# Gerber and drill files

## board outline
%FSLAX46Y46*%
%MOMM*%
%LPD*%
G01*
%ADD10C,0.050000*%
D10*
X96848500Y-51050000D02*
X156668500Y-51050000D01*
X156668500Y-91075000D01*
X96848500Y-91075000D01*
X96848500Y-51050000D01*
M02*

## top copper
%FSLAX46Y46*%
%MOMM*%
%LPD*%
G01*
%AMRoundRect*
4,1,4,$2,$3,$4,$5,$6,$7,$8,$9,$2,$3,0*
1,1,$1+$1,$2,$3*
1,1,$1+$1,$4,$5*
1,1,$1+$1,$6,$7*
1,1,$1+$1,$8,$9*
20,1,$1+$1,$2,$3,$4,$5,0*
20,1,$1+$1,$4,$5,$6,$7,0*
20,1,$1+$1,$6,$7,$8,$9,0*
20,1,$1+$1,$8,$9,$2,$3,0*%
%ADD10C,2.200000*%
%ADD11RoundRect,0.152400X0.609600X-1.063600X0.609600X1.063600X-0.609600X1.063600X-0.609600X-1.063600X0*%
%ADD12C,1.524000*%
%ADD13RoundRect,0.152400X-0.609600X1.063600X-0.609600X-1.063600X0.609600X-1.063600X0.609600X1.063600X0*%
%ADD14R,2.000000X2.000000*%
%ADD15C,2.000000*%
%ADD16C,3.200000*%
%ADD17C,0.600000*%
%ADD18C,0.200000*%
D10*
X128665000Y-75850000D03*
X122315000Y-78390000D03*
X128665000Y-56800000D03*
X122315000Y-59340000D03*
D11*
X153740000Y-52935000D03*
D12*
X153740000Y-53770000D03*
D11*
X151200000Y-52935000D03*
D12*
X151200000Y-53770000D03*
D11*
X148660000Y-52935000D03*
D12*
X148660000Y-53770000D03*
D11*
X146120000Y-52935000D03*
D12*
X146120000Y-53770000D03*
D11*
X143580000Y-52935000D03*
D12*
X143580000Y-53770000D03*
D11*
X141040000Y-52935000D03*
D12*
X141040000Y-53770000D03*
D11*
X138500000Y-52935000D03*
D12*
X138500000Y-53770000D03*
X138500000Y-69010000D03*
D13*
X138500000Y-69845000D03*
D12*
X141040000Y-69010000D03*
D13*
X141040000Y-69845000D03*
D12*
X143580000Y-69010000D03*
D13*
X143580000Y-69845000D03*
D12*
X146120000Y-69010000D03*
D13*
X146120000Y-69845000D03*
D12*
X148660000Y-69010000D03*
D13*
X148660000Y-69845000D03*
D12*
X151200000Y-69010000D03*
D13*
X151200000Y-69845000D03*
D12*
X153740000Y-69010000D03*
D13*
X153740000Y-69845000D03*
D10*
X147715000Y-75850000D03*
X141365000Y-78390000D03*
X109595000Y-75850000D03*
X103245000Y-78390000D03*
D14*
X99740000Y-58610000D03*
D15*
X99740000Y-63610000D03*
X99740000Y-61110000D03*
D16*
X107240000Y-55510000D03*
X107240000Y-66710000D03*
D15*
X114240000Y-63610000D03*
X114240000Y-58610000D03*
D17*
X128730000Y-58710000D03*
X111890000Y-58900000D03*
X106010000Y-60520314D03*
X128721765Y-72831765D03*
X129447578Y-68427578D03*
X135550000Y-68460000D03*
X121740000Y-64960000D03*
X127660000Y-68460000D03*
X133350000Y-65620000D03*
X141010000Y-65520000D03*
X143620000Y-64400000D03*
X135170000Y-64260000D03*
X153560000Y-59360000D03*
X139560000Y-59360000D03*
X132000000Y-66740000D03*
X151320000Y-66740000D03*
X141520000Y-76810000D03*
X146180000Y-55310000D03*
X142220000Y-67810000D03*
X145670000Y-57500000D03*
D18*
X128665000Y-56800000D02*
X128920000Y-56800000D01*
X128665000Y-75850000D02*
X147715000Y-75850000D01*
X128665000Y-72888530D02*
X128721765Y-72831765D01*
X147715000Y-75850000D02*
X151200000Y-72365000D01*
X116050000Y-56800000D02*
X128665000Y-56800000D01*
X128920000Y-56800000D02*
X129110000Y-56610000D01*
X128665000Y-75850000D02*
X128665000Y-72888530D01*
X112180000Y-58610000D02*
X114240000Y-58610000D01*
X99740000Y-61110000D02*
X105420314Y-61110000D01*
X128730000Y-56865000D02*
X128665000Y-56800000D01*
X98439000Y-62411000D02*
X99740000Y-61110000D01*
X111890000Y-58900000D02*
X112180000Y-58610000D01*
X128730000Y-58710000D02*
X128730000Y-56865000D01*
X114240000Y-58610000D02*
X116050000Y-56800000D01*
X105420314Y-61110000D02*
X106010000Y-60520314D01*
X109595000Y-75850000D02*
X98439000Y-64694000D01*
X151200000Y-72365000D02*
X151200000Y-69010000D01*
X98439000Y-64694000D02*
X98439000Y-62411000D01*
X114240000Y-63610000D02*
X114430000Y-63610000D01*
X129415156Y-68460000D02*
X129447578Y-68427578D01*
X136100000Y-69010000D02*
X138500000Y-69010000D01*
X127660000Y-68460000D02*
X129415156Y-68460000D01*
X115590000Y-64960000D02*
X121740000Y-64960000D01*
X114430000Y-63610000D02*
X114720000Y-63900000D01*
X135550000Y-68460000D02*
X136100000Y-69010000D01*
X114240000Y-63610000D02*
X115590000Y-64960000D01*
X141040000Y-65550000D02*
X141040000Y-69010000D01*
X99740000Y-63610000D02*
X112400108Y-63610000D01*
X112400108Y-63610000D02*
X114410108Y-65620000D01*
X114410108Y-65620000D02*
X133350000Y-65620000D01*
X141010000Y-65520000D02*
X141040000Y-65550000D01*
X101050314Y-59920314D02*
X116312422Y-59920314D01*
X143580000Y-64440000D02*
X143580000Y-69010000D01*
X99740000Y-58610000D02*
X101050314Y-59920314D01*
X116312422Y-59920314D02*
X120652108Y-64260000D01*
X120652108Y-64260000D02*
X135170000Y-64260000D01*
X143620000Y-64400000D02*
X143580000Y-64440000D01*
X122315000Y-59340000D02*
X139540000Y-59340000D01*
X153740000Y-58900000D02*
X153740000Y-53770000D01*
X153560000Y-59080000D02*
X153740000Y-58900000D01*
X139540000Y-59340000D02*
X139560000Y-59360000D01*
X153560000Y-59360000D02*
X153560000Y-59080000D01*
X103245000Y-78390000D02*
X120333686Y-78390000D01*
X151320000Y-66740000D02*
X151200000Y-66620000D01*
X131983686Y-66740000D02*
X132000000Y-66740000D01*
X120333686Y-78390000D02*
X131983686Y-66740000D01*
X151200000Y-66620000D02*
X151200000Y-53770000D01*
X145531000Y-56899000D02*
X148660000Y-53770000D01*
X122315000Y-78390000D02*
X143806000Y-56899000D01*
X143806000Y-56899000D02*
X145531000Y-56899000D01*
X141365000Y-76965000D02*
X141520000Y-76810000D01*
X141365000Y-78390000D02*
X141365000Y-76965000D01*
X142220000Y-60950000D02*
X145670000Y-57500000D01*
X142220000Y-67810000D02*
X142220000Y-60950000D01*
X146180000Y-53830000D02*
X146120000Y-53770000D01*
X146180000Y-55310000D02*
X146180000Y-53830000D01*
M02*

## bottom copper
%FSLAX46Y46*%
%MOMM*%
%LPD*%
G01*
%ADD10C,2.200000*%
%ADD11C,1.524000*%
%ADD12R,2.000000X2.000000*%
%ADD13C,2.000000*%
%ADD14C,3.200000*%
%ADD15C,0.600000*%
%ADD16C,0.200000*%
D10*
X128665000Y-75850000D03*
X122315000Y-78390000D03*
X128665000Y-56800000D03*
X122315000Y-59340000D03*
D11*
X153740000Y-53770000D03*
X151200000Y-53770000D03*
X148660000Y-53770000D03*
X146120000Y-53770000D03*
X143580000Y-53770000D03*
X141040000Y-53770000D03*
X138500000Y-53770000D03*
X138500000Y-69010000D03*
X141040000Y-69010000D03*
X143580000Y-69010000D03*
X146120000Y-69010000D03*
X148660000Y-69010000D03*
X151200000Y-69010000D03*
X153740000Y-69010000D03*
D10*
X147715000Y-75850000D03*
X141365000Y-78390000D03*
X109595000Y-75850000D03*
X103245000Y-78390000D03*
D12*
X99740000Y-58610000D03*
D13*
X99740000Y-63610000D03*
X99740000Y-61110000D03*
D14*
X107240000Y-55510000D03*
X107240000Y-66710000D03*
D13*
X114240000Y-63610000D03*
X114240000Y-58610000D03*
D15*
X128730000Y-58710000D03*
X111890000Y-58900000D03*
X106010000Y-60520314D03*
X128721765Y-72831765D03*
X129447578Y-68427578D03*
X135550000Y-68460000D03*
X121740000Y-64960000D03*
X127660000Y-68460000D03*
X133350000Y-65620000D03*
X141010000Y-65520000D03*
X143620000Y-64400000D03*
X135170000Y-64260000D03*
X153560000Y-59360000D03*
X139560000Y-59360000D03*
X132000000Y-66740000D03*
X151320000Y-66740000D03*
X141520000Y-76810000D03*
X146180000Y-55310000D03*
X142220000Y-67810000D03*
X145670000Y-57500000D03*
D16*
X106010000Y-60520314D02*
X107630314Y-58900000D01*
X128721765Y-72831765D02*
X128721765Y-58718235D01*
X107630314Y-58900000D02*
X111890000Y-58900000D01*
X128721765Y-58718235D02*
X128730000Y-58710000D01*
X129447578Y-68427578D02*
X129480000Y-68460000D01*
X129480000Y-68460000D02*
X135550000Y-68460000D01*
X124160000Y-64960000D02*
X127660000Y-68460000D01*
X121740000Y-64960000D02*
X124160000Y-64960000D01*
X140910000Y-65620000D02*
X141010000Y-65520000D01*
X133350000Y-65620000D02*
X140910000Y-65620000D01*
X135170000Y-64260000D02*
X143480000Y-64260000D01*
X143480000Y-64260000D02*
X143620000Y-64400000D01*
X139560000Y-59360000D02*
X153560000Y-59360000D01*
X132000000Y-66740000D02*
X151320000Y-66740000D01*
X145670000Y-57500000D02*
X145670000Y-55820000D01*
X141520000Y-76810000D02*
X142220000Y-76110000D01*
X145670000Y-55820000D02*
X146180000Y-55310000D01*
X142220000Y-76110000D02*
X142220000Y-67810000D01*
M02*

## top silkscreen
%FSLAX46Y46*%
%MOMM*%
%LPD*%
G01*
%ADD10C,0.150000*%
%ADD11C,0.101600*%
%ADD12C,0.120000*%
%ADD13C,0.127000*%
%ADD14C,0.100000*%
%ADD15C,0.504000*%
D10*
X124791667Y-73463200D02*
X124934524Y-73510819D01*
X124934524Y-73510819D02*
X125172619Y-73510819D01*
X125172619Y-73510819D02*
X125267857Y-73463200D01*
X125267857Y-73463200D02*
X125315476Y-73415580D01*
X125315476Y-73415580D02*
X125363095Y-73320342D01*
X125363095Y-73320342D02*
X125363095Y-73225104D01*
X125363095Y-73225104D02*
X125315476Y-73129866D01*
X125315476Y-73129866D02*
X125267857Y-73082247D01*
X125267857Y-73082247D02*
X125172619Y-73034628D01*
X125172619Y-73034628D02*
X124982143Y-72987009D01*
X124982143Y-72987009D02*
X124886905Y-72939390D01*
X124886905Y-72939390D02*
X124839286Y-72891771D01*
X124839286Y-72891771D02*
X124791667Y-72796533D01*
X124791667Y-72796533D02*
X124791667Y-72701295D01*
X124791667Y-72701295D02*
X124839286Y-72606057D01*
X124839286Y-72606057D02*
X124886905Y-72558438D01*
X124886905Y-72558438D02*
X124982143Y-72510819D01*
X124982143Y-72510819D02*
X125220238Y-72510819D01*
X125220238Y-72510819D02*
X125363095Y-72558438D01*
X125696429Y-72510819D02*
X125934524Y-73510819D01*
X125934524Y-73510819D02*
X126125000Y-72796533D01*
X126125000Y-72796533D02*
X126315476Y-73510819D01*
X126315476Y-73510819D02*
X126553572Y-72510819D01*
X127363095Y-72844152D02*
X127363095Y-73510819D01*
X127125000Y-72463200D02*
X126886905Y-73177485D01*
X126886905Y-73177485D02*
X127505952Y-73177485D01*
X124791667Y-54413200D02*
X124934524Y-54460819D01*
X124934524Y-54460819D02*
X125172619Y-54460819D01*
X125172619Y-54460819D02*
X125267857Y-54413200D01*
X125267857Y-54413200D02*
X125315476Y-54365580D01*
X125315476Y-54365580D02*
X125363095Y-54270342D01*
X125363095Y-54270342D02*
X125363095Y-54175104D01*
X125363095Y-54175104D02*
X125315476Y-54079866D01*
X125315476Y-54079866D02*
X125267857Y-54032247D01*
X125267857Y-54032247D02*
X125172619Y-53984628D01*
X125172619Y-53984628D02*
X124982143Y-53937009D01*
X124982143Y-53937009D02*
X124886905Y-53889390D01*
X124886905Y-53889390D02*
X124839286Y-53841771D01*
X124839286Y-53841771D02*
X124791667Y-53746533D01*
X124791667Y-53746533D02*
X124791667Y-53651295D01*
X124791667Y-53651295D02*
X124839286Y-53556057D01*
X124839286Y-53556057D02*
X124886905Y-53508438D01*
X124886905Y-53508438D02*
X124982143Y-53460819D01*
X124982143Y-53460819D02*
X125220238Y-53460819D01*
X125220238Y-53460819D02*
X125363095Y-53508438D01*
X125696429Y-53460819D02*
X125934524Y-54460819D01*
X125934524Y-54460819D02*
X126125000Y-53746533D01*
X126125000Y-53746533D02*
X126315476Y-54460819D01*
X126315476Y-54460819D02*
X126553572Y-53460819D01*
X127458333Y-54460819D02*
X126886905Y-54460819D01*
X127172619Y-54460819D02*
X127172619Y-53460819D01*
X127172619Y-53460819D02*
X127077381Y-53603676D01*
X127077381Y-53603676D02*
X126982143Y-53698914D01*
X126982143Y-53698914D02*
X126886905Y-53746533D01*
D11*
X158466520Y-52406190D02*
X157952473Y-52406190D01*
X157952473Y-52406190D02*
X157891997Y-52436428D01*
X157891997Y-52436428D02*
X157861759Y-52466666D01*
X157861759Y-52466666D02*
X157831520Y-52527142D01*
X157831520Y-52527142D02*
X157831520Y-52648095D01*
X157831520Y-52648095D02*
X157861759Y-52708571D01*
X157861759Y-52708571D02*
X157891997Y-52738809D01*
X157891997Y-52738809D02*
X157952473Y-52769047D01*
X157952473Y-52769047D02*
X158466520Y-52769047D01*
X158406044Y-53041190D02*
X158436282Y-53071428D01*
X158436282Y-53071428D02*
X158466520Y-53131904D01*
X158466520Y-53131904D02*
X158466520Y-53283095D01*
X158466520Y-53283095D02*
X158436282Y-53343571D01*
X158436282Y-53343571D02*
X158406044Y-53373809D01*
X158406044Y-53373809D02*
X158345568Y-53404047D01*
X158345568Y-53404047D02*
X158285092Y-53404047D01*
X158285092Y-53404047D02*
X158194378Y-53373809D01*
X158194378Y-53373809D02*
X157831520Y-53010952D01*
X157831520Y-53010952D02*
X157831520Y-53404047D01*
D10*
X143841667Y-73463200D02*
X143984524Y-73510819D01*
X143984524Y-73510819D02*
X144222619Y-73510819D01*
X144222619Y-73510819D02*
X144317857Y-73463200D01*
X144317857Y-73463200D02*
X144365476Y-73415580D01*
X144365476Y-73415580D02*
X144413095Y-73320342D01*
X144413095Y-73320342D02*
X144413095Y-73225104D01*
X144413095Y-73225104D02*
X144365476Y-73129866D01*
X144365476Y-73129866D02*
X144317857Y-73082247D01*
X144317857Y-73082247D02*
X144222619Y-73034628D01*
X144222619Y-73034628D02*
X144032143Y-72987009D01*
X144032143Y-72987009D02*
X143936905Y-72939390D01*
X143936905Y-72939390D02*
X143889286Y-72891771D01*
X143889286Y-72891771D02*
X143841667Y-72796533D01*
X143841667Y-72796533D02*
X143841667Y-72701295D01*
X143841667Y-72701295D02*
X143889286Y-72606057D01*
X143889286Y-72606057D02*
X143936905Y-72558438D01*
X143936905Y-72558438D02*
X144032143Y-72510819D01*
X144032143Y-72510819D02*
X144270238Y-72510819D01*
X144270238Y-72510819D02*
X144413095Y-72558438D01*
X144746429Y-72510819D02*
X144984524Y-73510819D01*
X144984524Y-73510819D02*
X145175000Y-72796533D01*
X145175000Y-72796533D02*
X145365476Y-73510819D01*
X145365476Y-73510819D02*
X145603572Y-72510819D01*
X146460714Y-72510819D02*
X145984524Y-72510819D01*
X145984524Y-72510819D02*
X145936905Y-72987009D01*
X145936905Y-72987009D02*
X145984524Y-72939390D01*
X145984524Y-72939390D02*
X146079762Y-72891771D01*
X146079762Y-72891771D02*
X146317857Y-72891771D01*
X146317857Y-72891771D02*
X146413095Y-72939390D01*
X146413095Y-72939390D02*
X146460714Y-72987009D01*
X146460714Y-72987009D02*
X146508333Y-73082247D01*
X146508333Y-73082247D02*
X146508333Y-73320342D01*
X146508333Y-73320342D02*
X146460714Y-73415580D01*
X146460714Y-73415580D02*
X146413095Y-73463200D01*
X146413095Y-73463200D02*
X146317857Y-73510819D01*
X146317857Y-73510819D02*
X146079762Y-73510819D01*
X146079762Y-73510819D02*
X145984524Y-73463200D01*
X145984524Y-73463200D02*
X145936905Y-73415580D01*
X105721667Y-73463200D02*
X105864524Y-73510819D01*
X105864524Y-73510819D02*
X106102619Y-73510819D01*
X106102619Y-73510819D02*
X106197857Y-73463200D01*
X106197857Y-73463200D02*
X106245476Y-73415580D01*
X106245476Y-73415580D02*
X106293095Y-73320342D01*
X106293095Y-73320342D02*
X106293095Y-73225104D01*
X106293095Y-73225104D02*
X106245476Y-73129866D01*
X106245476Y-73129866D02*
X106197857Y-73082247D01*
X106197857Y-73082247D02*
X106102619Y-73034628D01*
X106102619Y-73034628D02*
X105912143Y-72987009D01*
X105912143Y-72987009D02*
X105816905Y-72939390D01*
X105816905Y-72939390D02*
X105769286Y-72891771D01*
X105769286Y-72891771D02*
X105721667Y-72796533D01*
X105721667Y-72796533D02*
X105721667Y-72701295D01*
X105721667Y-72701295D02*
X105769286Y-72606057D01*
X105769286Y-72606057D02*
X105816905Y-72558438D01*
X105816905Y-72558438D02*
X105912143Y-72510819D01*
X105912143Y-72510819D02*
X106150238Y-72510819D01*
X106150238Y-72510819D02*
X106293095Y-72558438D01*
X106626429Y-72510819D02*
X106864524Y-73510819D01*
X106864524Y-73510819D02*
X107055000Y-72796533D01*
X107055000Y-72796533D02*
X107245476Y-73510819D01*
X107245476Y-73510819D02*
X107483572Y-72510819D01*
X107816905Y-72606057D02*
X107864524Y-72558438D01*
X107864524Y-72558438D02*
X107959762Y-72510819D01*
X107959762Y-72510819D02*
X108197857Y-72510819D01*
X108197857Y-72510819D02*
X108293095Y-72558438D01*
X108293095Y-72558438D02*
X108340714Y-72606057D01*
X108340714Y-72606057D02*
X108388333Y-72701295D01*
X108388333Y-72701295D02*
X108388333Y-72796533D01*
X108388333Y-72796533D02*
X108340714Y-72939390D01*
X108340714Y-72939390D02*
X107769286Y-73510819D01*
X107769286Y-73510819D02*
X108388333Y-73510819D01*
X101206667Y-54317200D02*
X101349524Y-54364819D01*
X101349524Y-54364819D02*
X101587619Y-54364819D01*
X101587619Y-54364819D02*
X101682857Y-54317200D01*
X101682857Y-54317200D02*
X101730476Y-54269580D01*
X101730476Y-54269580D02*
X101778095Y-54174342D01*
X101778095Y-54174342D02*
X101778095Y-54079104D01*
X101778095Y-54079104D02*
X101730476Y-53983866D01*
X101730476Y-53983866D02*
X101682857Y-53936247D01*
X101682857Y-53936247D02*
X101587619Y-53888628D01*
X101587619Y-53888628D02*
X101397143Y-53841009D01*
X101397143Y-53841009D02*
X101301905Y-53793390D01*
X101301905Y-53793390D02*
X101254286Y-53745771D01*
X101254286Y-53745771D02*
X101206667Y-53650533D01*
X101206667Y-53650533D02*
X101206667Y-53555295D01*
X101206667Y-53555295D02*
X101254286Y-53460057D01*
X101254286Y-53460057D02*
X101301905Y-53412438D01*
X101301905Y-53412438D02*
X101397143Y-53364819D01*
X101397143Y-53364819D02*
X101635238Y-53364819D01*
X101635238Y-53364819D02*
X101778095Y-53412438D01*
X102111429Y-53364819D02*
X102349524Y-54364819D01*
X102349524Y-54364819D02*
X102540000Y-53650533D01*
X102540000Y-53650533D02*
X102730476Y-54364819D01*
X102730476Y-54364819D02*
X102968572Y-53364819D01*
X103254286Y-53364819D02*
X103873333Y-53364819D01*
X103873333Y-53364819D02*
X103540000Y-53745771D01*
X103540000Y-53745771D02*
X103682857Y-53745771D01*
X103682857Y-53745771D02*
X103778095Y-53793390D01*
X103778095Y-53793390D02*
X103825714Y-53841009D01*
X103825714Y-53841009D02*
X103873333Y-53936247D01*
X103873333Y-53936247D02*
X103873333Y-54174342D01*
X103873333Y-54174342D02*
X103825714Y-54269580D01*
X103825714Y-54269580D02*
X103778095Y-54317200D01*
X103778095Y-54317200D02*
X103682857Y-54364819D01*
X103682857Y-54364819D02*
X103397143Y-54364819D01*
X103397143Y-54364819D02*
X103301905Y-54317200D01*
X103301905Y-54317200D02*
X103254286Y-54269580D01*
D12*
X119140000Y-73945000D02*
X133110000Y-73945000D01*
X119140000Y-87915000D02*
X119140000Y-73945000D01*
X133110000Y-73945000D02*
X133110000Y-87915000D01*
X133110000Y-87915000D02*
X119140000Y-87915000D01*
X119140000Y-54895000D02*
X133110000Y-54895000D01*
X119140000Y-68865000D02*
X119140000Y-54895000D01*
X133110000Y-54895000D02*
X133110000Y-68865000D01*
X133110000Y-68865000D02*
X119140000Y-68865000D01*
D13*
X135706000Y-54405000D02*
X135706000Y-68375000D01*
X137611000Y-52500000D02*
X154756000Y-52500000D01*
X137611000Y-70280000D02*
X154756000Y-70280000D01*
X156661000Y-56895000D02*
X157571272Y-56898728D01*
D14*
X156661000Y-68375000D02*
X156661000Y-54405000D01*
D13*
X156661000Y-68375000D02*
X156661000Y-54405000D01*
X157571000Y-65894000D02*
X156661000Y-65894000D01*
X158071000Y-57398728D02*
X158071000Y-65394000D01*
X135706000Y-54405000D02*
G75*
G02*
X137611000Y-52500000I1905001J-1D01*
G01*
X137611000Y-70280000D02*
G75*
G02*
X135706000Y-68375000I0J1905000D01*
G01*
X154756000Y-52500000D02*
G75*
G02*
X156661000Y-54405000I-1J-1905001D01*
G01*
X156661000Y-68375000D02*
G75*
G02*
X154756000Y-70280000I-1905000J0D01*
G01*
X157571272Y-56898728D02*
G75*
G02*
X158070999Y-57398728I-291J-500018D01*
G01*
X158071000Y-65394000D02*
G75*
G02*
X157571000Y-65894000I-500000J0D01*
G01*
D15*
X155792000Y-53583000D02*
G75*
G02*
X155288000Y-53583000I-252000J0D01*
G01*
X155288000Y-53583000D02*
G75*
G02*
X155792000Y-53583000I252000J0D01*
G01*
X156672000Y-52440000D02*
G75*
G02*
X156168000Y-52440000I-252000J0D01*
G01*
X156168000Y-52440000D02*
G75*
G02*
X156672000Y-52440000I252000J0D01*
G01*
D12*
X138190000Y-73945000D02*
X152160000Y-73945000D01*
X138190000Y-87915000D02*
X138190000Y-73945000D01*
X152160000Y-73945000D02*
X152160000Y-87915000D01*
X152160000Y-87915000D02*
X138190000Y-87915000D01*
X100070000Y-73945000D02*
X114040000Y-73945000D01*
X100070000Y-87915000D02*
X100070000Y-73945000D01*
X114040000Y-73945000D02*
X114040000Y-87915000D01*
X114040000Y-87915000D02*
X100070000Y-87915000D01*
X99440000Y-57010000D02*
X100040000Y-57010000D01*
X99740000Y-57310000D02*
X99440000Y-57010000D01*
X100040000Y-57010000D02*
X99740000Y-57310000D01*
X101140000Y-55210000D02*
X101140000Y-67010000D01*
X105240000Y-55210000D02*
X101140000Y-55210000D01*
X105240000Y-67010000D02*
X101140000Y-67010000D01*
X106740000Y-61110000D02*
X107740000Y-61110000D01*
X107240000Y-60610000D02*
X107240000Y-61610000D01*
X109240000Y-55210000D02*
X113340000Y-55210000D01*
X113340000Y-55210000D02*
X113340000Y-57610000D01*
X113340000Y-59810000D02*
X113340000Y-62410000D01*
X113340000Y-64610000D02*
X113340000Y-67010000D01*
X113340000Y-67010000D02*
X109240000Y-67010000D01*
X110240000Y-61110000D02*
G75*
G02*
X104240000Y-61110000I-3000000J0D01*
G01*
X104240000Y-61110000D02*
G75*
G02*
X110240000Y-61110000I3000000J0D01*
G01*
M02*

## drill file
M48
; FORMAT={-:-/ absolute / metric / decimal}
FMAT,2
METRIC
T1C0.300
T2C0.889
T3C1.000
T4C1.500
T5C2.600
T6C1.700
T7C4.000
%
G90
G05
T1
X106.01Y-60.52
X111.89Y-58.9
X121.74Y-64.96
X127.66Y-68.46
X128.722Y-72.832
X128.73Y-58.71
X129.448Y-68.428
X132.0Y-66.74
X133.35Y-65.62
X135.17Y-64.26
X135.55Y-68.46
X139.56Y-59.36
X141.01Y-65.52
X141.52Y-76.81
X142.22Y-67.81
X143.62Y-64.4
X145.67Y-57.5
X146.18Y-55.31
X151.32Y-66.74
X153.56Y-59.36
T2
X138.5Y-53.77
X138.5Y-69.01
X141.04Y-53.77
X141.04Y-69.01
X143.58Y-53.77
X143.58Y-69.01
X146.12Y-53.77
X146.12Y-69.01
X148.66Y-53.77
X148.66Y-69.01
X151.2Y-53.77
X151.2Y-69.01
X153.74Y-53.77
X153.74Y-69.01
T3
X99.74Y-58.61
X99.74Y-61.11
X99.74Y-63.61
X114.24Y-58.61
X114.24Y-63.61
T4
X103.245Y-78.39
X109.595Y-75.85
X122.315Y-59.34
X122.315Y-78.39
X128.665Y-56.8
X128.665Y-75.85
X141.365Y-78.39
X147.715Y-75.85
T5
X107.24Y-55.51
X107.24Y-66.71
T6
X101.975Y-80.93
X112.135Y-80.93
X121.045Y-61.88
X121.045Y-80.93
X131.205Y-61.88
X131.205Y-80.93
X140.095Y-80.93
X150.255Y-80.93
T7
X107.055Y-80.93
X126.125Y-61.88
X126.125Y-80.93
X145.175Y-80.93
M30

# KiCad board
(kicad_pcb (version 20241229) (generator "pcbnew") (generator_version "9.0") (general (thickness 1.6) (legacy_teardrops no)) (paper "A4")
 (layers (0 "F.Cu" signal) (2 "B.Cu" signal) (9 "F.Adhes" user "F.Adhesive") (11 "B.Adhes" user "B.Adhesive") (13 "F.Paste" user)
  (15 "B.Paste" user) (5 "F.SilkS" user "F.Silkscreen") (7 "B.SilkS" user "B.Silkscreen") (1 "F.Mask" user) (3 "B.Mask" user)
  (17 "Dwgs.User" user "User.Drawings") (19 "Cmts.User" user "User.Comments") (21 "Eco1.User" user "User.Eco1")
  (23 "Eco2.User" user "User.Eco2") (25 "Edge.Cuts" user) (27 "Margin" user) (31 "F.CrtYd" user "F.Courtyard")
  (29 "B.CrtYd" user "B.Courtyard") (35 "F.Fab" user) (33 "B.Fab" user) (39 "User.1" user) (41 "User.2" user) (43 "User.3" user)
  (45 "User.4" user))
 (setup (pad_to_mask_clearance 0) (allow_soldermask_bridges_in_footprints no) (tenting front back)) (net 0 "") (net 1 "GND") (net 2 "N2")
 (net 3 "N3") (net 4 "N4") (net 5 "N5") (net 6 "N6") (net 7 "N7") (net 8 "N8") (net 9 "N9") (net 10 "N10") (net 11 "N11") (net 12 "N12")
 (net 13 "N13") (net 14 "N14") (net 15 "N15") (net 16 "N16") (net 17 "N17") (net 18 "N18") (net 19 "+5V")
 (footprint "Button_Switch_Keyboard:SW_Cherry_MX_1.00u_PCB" (layer "F.Cu") (at 128.665 75.85)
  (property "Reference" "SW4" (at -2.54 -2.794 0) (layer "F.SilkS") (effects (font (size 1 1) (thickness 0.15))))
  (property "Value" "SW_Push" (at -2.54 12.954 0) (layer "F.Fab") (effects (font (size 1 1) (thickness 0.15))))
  (fp_line (start -9.525 -1.905) (end 4.445 -1.905) (stroke (width 0.12) (type solid)) (layer "F.SilkS"))
  (fp_line (start -9.525 12.065) (end -9.525 -1.905) (stroke (width 0.12) (type solid)) (layer "F.SilkS"))
  (fp_line (start 4.445 -1.905) (end 4.445 12.065) (stroke (width 0.12) (type solid)) (layer "F.SilkS"))
  (fp_line (start 4.445 12.065) (end -9.525 12.065) (stroke (width 0.12) (type solid)) (layer "F.SilkS"))
  (pad "" np_thru_hole circle (at -7.62 5.08) (size 1.7 1.7) (drill 1.7) (layers "*.Cu" "*.Mask"))
  (pad "" np_thru_hole circle (at -2.54 5.08) (size 4 4) (drill 4) (layers "*.Cu" "*.Mask"))
  (pad "" np_thru_hole circle (at 2.54 5.08) (size 1.7 1.7) (drill 1.7) (layers "*.Cu" "*.Mask"))
  (pad "1" thru_hole circle (at 0 0) (size 2.2 2.2) (drill 1.5) (layers "*.Cu" "*.Mask") (remove_unused_layers no) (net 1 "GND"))
  (pad "2" thru_hole circle (at -6.35 2.54) (size 2.2 2.2) (drill 1.5) (layers "*.Cu" "*.Mask") (remove_unused_layers no) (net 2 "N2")))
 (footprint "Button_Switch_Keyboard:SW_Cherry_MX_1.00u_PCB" (layer "F.Cu") (at 128.665 56.8)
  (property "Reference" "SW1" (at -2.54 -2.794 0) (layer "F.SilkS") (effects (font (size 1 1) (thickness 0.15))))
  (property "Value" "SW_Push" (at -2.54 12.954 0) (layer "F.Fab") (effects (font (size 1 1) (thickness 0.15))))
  (fp_line (start -9.525 -1.905) (end 4.445 -1.905) (stroke (width 0.12) (type solid)) (layer "F.SilkS"))
  (fp_line (start -9.525 12.065) (end -9.525 -1.905) (stroke (width 0.12) (type solid)) (layer "F.SilkS"))
  (fp_line (start 4.445 -1.905) (end 4.445 12.065) (stroke (width 0.12) (type solid)) (layer "F.SilkS"))
  (fp_line (start 4.445 12.065) (end -9.525 12.065) (stroke (width 0.12) (type solid)) (layer "F.SilkS"))
  (pad "" np_thru_hole circle (at -7.62 5.08) (size 1.7 1.7) (drill 1.7) (layers "*.Cu" "*.Mask"))
  (pad "" np_thru_hole circle (at -2.54 5.08) (size 4 4) (drill 4) (layers "*.Cu" "*.Mask"))
  (pad "" np_thru_hole circle (at 2.54 5.08) (size 1.7 1.7) (drill 1.7) (layers "*.Cu" "*.Mask"))
  (pad "1" thru_hole circle (at 0 0) (size 2.2 2.2) (drill 1.5) (layers "*.Cu" "*.Mask") (remove_unused_layers no) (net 1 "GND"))
  (pad "2" thru_hole circle (at -6.35 2.54) (size 2.2 2.2) (drill 1.5) (layers "*.Cu" "*.Mask") (remove_unused_layers no) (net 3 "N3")))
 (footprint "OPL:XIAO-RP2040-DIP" (layer "F.Cu") (at 146.12 61.39 -90)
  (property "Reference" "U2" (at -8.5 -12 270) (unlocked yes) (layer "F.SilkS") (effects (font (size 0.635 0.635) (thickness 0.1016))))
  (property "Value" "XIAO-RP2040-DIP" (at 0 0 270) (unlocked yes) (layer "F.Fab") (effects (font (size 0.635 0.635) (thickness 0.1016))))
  (fp_line (start -6.985 10.414) (end 6.985 10.414) (stroke (width 0.127) (type solid)) (layer "F.SilkS"))
  (fp_line (start -8.89 8.509) (end -8.89 -8.636) (stroke (width 0.127) (type solid)) (layer "F.SilkS"))
  (fp_line (start 8.89 8.509) (end 8.89 -8.636) (stroke (width 0.127) (type solid)) (layer "F.SilkS"))
  (fp_line (start -4.495 -10.541) (end -4.491272 -11.451272) (stroke (width 0.127) (type solid)) (layer "F.SilkS"))
  (fp_line (start 6.985 -10.541) (end -6.985 -10.541) (stroke (width 0.1) (type solid)) (layer "F.SilkS"))
  (fp_line (start 6.985 -10.541) (end -6.985 -10.541) (stroke (width 0.127) (type solid)) (layer "F.SilkS"))
  (fp_line (start 4.504 -11.451) (end 4.504 -10.541) (stroke (width 0.127) (type solid)) (layer "F.SilkS"))
  (fp_line (start -3.991272 -11.951) (end 4.004 -11.951) (stroke (width 0.127) (type solid)) (layer "F.SilkS"))
  (fp_arc (start -6.985 10.414) (mid -8.332038 9.856038) (end -8.89 8.509) (stroke (width 0.127) (type solid)) (layer "F.SilkS"))
  (fp_arc (start 8.89 8.509) (mid 8.332038 9.856038) (end 6.985 10.414) (stroke (width 0.127) (type solid)) (layer "F.SilkS"))
  (fp_arc (start -8.89 -8.636) (mid -8.332038 -9.983038) (end -6.985 -10.541) (stroke (width 0.127) (type solid)) (layer "F.SilkS"))
  (fp_arc (start 6.985 -10.541) (mid 8.332038 -9.983038) (end 8.89 -8.636) (stroke (width 0.127) (type solid)) (layer "F.SilkS"))
  (fp_arc (start -4.491272 -11.451272) (mid -4.344728 -11.80464) (end -3.991272 -11.951) (stroke (width 0.127) (type default))
   (layer "F.SilkS"))
  (fp_arc (start 4.004 -11.951) (mid 4.357553 -11.804553) (end 4.504 -11.451) (stroke (width 0.127) (type default)) (layer "F.SilkS"))
  (fp_circle (center -7.807 -9.42) (end -7.807 -9.674) (stroke (width 0.5) (type solid)) (fill yes) (layer "F.SilkS"))
  (fp_circle (center -8.95 -10.3) (end -8.95 -10.554) (stroke (width 0.5) (type solid)) (fill yes) (layer "F.SilkS"))
  (pad "1" smd roundrect (at -8.455 -7.62 90) (size 2.432 1.524) (layers "F.Cu" "F.Mask") (roundrect_rratio 0.1) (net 3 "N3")
   (thermal_bridge_angle 45))
  (pad "1" thru_hole circle (at -7.62 -7.62 90) (size 1.524 1.524) (drill 0.889) (layers "*.Cu" "*.Mask") (remove_unused_layers no)
   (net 3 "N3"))
  (pad "2" smd roundrect (at -8.455 -5.08 90) (size 2.432 1.524) (layers "F.Cu" "F.Mask") (roundrect_rratio 0.1) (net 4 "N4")
   (thermal_bridge_angle 45))
  (pad "2" thru_hole circle (at -7.62 -5.08 90) (size 1.524 1.524) (drill 0.889) (layers "*.Cu" "*.Mask") (remove_unused_layers no)
   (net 4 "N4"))
  (pad "3" smd roundrect (at -8.455 -2.54 90) (size 2.432 1.524) (layers "F.Cu" "F.Mask") (roundrect_rratio 0.1) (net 2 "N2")
   (thermal_bridge_angle 45))
  (pad "3" thru_hole circle (at -7.62 -2.54 90) (size 1.524 1.524) (drill 0.889) (layers "*.Cu" "*.Mask") (remove_unused_layers no)
   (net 2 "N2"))
  (pad "4" smd roundrect (at -8.455 0 90) (size 2.432 1.524) (layers "F.Cu" "F.Mask") (roundrect_rratio 0.1) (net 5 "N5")
   (thermal_bridge_angle 45))
  (pad "4" thru_hole circle (at -7.62 0 90) (size 1.524 1.524) (drill 0.889) (layers "*.Cu" "*.Mask") (remove_unused_layers no) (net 5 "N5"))
  (pad "5" smd roundrect (at -8.455 2.54 90) (size 2.432 1.524) (layers "F.Cu" "F.Mask") (roundrect_rratio 0.1) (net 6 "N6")
   (thermal_bridge_angle 45))
  (pad "5" thru_hole circle (at -7.62 2.54 90) (size 1.524 1.524) (drill 0.889) (layers "*.Cu" "*.Mask") (remove_unused_layers no)
   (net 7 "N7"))
  (pad "6" smd roundrect (at -8.455 5.08 90) (size 2.432 1.524) (layers "F.Cu" "F.Mask") (roundrect_rratio 0.1) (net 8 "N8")
   (thermal_bridge_angle 45))
  (pad "6" thru_hole circle (at -7.62 5.08 90) (size 1.524 1.524) (drill 0.889) (layers "*.Cu" "*.Mask") (remove_unused_layers no)
   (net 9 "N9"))
  (pad "7" smd roundrect (at -8.455 7.62 90) (size 2.432 1.524) (layers "F.Cu" "F.Mask") (roundrect_rratio 0.1) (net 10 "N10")
   (thermal_bridge_angle 45))
  (pad "7" thru_hole circle (at -7.62 7.62 90) (size 1.524 1.524) (drill 0.889) (layers "*.Cu" "*.Mask") (remove_unused_layers no)
   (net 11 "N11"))
  (pad "8" thru_hole circle (at 7.62 7.62 270) (size 1.524 1.524) (drill 0.889) (layers "*.Cu" "*.Mask") (remove_unused_layers no)
   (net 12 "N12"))
  (pad "8" smd roundrect (at 8.455 7.62 270) (size 2.432 1.524) (layers "F.Cu" "F.Mask") (roundrect_rratio 0.1) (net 12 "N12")
   (thermal_bridge_angle 45))
  (pad "9" thru_hole circle (at 7.62 5.08 270) (size 1.524 1.524) (drill 0.889) (layers "*.Cu" "*.Mask") (remove_unused_layers no)
   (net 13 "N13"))
  (pad "9" smd roundrect (at 8.455 5.08 270) (size 2.432 1.524) (layers "F.Cu" "F.Mask") (roundrect_rratio 0.1) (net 13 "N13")
   (thermal_bridge_angle 45))
  (pad "10" thru_hole circle (at 7.62 2.54 270) (size 1.524 1.524) (drill 0.889) (layers "*.Cu" "*.Mask") (remove_unused_layers no)
   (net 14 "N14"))
  (pad "10" smd roundrect (at 8.455 2.54 270) (size 2.432 1.524) (layers "F.Cu" "F.Mask") (roundrect_rratio 0.1) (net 14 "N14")
   (thermal_bridge_angle 45))
  (pad "11" thru_hole circle (at 7.62 0 270) (size 1.524 1.524) (drill 0.889) (layers "*.Cu" "*.Mask") (remove_unused_layers no)
   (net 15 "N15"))
  (pad "11" smd roundrect (at 8.455 0 270) (size 2.432 1.524) (layers "F.Cu" "F.Mask") (roundrect_rratio 0.1) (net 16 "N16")
   (thermal_bridge_angle 45))
  (pad "12" thru_hole circle (at 7.62 -2.54 270) (size 1.524 1.524) (drill 0.889) (layers "*.Cu" "*.Mask") (remove_unused_layers no)
   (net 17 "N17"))
  (pad "12" smd roundrect (at 8.455 -2.54 270) (size 2.432 1.524) (layers "F.Cu" "F.Mask") (roundrect_rratio 0.1) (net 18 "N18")
   (thermal_bridge_angle 45))
  (pad "13" thru_hole circle (at 7.62 -5.08 270) (size 1.524 1.524) (drill 0.889) (layers "*.Cu" "*.Mask") (remove_unused_layers no)
   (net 1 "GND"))
  (pad "13" smd roundrect (at 8.455 -5.08 270) (size 2.432 1.524) (layers "F.Cu" "F.Mask") (roundrect_rratio 0.1) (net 1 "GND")
   (thermal_bridge_angle 45))
  (pad "14" thru_hole circle (at 7.62 -7.62 270) (size 1.524 1.524) (drill 0.889) (layers "*.Cu" "*.Mask") (remove_unused_layers no)
   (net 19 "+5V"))
  (pad "14" smd roundrect (at 8.455 -7.62 270) (size 2.432 1.524) (layers "F.Cu" "F.Mask") (roundrect_rratio 0.1) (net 19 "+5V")
   (thermal_bridge_angle 45)))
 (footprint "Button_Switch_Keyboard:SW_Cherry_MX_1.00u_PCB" (layer "F.Cu") (at 147.715 75.85)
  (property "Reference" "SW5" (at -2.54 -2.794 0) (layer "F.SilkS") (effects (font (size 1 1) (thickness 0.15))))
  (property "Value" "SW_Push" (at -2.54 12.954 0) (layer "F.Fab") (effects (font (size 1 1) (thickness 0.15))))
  (fp_line (start -9.525 -1.905) (end 4.445 -1.905) (stroke (width 0.12) (type solid)) (layer "F.SilkS"))
  (fp_line (start -9.525 12.065) (end -9.525 -1.905) (stroke (width 0.12) (type solid)) (layer "F.SilkS"))
  (fp_line (start 4.445 -1.905) (end 4.445 12.065) (stroke (width 0.12) (type solid)) (layer "F.SilkS"))
  (fp_line (start 4.445 12.065) (end -9.525 12.065) (stroke (width 0.12) (type solid)) (layer "F.SilkS"))
  (pad "" np_thru_hole circle (at -7.62 5.08) (size 1.7 1.7) (drill 1.7) (layers "*.Cu" "*.Mask"))
  (pad "" np_thru_hole circle (at -2.54 5.08) (size 4 4) (drill 4) (layers "*.Cu" "*.Mask"))
  (pad "" np_thru_hole circle (at 2.54 5.08) (size 1.7 1.7) (drill 1.7) (layers "*.Cu" "*.Mask"))
  (pad "1" thru_hole circle (at 0 0) (size 2.2 2.2) (drill 1.5) (layers "*.Cu" "*.Mask") (remove_unused_layers no) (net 1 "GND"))
  (pad "2" thru_hole circle (at -6.35 2.54) (size 2.2 2.2) (drill 1.5) (layers "*.Cu" "*.Mask") (remove_unused_layers no) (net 5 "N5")))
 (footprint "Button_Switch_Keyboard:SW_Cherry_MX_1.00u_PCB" (layer "F.Cu") (at 109.595 75.85)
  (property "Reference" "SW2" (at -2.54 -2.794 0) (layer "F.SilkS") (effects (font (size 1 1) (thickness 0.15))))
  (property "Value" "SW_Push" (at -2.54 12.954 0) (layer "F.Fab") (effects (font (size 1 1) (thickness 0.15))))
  (fp_line (start -9.525 -1.905) (end 4.445 -1.905) (stroke (width 0.12) (type solid)) (layer "F.SilkS"))
  (fp_line (start -9.525 12.065) (end -9.525 -1.905) (stroke (width 0.12) (type solid)) (layer "F.SilkS"))
  (fp_line (start 4.445 -1.905) (end 4.445 12.065) (stroke (width 0.12) (type solid)) (layer "F.SilkS"))
  (fp_line (start 4.445 12.065) (end -9.525 12.065) (stroke (width 0.12) (type solid)) (layer "F.SilkS"))
  (pad "" np_thru_hole circle (at -7.62 5.08) (size 1.7 1.7) (drill 1.7) (layers "*.Cu" "*.Mask"))
  (pad "" np_thru_hole circle (at -2.54 5.08) (size 4 4) (drill 4) (layers "*.Cu" "*.Mask"))
  (pad "" np_thru_hole circle (at 2.54 5.08) (size 1.7 1.7) (drill 1.7) (layers "*.Cu" "*.Mask"))
  (pad "1" thru_hole circle (at 0 0) (size 2.2 2.2) (drill 1.5) (layers "*.Cu" "*.Mask") (remove_unused_layers no) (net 1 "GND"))
  (pad "2" thru_hole circle (at -6.35 2.54) (size 2.2 2.2) (drill 1.5) (layers "*.Cu" "*.Mask") (remove_unused_layers no) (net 4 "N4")))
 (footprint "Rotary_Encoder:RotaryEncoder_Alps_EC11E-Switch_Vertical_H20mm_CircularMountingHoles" (layer "F.Cu") (at 99.74 58.61)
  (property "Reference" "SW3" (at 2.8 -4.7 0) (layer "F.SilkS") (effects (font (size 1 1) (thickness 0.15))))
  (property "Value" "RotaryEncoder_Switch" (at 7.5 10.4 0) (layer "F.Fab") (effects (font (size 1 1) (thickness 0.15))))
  (fp_line (start -0.3 -1.6) (end 0.3 -1.6) (stroke (width 0.12) (type solid)) (layer "F.SilkS"))
  (fp_line (start 0 -1.3) (end -0.3 -1.6) (stroke (width 0.12) (type solid)) (layer "F.SilkS"))
  (fp_line (start 0.3 -1.6) (end 0 -1.3) (stroke (width 0.12) (type solid)) (layer "F.SilkS"))
  (fp_line (start 1.4 -3.4) (end 1.4 8.4) (stroke (width 0.12) (type solid)) (layer "F.SilkS"))
  (fp_line (start 5.5 -3.4) (end 1.4 -3.4) (stroke (width 0.12) (type solid)) (layer "F.SilkS"))
  (fp_line (start 5.5 8.4) (end 1.4 8.4) (stroke (width 0.12) (type solid)) (layer "F.SilkS"))
  (fp_line (start 7 2.5) (end 8 2.5) (stroke (width 0.12) (type solid)) (layer "F.SilkS"))
  (fp_line (start 7.5 2) (end 7.5 3) (stroke (width 0.12) (type solid)) (layer "F.SilkS"))
  (fp_line (start 9.5 -3.4) (end 13.6 -3.4) (stroke (width 0.12) (type solid)) (layer "F.SilkS"))
  (fp_line (start 13.6 -3.4) (end 13.6 -1) (stroke (width 0.12) (type solid)) (layer "F.SilkS"))
  (fp_line (start 13.6 1.2) (end 13.6 3.8) (stroke (width 0.12) (type solid)) (layer "F.SilkS"))
  (fp_line (start 13.6 6) (end 13.6 8.4) (stroke (width 0.12) (type solid)) (layer "F.SilkS"))
  (fp_line (start 13.6 8.4) (end 9.5 8.4) (stroke (width 0.12) (type solid)) (layer "F.SilkS"))
  (fp_circle (center 7.5 2.5) (end 10.5 2.5) (stroke (width 0.12) (type solid)) (fill no) (layer "F.SilkS"))
  (pad "A" thru_hole rect (at 0 0) (size 2 2) (drill 1) (layers "*.Cu" "*.Mask") (remove_unused_layers no) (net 14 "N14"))
  (pad "B" thru_hole circle (at 0 5) (size 2 2) (drill 1) (layers "*.Cu" "*.Mask") (remove_unused_layers no) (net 13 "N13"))
  (pad "C" thru_hole circle (at 0 2.5) (size 2 2) (drill 1) (layers "*.Cu" "*.Mask") (remove_unused_layers no) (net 1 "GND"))
  (pad "MP" thru_hole circle (at 7.5 -3.1) (size 3.2 3.2) (drill 2.6) (layers "*.Cu" "*.Mask") (remove_unused_layers no))
  (pad "MP" thru_hole circle (at 7.5 8.1) (size 3.2 3.2) (drill 2.6) (layers "*.Cu" "*.Mask") (remove_unused_layers no))
  (pad "S1" thru_hole circle (at 14.5 5) (size 2 2) (drill 1) (layers "*.Cu" "*.Mask") (remove_unused_layers no) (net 12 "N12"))
  (pad "S2" thru_hole circle (at 14.5 0) (size 2 2) (drill 1) (layers "*.Cu" "*.Mask") (remove_unused_layers no) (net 1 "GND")))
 (gr_rect (start 96.8485 51.05) (end 156.6685 91.075) (stroke (width 0.05) (type default)) (fill no) (layer "Edge.Cuts"))
 (segment (start 128.665 56.8) (end 128.92 56.8) (width 0.2) (layer "F.Cu") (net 1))
 (segment (start 128.665 75.85) (end 147.715 75.85) (width 0.2) (layer "F.Cu") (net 1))
 (segment (start 128.665 72.88853) (end 128.721765 72.831765) (width 0.2) (layer "F.Cu") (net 1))
 (segment (start 147.715 75.85) (end 151.2 72.365) (width 0.2) (layer "F.Cu") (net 1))
 (segment (start 116.05 56.8) (end 128.665 56.8) (width 0.2) (layer "F.Cu") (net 1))
 (segment (start 128.92 56.8) (end 129.11 56.61) (width 0.2) (layer "F.Cu") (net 1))
 (segment (start 128.665 75.85) (end 128.665 72.88853) (width 0.2) (layer "F.Cu") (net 1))
 (segment (start 112.18 58.61) (end 114.24 58.61) (width 0.2) (layer "F.Cu") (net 1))
 (segment (start 99.74 61.11) (end 105.420314 61.11) (width 0.2) (layer "F.Cu") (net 1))
 (segment (start 128.73 56.865) (end 128.665 56.8) (width 0.2) (layer "F.Cu") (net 1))
 (segment (start 98.439 62.411) (end 99.74 61.11) (width 0.2) (layer "F.Cu") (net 1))
 (segment (start 111.89 58.9) (end 112.18 58.61) (width 0.2) (layer "F.Cu") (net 1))
 (segment (start 128.73 58.71) (end 128.73 56.865) (width 0.2) (layer "F.Cu") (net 1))
 (segment (start 114.24 58.61) (end 116.05 56.8) (width 0.2) (layer "F.Cu") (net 1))
 (segment (start 105.420314 61.11) (end 106.01 60.520314) (width 0.2) (layer "F.Cu") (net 1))
 (segment (start 109.595 75.85) (end 98.439 64.694) (width 0.2) (layer "F.Cu") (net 1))
 (segment (start 151.2 72.365) (end 151.2 69.01) (width 0.2) (layer "F.Cu") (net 1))
 (segment (start 98.439 64.694) (end 98.439 62.411) (width 0.2) (layer "F.Cu") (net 1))
 (via (at 128.73 58.71) (size 0.6) (drill 0.3) (layers "F.Cu" "B.Cu") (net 1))
 (via (at 111.89 58.9) (size 0.6) (drill 0.3) (layers "F.Cu" "B.Cu") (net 1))
 (via (at 106.01 60.520314) (size 0.6) (drill 0.3) (layers "F.Cu" "B.Cu") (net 1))
 (via (at 128.721765 72.831765) (size 0.6) (drill 0.3) (layers "F.Cu" "B.Cu") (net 1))
 (segment (start 106.01 60.520314) (end 107.630314 58.9) (width 0.2) (layer "B.Cu") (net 1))
 (segment (start 128.721765 72.831765) (end 128.721765 58.718235) (width 0.2) (layer "B.Cu") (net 1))
 (segment (start 107.630314 58.9) (end 111.89 58.9) (width 0.2) (layer "B.Cu") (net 1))
 (segment (start 128.721765 58.718235) (end 128.73 58.71) (width 0.2) (layer "B.Cu") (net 1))
 (segment (start 114.24 63.61) (end 114.43 63.61) (width 0.2) (layer "F.Cu") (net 12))
 (segment (start 129.415156 68.46) (end 129.447578 68.427578) (width 0.2) (layer "F.Cu") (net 12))
 (segment (start 136.1 69.01) (end 138.5 69.01) (width 0.2) (layer "F.Cu") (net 12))
 (segment (start 127.66 68.46) (end 129.415156 68.46) (width 0.2) (layer "F.Cu") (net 12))
 (segment (start 115.59 64.96) (end 121.74 64.96) (width 0.2) (layer "F.Cu") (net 12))
 (segment (start 114.43 63.61) (end 114.72 63.9) (width 0.2) (layer "F.Cu") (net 12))
 (segment (start 135.55 68.46) (end 136.1 69.01) (width 0.2) (layer "F.Cu") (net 12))
 (segment (start 114.24 63.61) (end 115.59 64.96) (width 0.2) (layer "F.Cu") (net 12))
 (via (at 129.447578 68.427578) (size 0.6) (drill 0.3) (layers "F.Cu" "B.Cu") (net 12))
 (via (at 135.55 68.46) (size 0.6) (drill 0.3) (layers "F.Cu" "B.Cu") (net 12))
 (via (at 121.74 64.96) (size 0.6) (drill 0.3) (layers "F.Cu" "B.Cu") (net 12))
 (via (at 127.66 68.46) (size 0.6) (drill 0.3) (layers "F.Cu" "B.Cu") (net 12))
 (segment (start 129.447578 68.427578) (end 129.48 68.46) (width 0.2) (layer "B.Cu") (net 12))
 (segment (start 129.48 68.46) (end 135.55 68.46) (width 0.2) (layer "B.Cu") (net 12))
 (segment (start 124.16 64.96) (end 127.66 68.46) (width 0.2) (layer "B.Cu") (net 12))
 (segment (start 121.74 64.96) (end 124.16 64.96) (width 0.2) (layer "B.Cu") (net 12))
 (segment (start 141.04 65.55) (end 141.04 69.01) (width 0.2) (layer "F.Cu") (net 13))
 (segment (start 99.74 63.61) (end 112.400108 63.61) (width 0.2) (layer "F.Cu") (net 13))
 (segment (start 112.400108 63.61) (end 114.410108 65.62) (width 0.2) (layer "F.Cu") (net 13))
 (segment (start 114.410108 65.62) (end 133.35 65.62) (width 0.2) (layer "F.Cu") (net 13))
 (segment (start 141.01 65.52) (end 141.04 65.55) (width 0.2) (layer "F.Cu") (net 13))
 (via (at 133.35 65.62) (size 0.6) (drill 0.3) (layers "F.Cu" "B.Cu") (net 13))
 (via (at 141.01 65.52) (size 0.6) (drill 0.3) (layers "F.Cu" "B.Cu") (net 13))
 (segment (start 140.91 65.62) (end 141.01 65.52) (width 0.2) (layer "B.Cu") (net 13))
 (segment (start 133.35 65.62) (end 140.91 65.62) (width 0.2) (layer "B.Cu") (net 13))
 (segment (start 101.050314 59.920314) (end 116.312422 59.920314) (width 0.2) (layer "F.Cu") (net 14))
 (segment (start 143.58 64.44) (end 143.58 69.01) (width 0.2) (layer "F.Cu") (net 14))
 (segment (start 99.74 58.61) (end 101.050314 59.920314) (width 0.2) (layer "F.Cu") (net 14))
 (segment (start 116.312422 59.920314) (end 120.652108 64.26) (width 0.2) (layer "F.Cu") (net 14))
 (segment (start 120.652108 64.26) (end 135.17 64.26) (width 0.2) (layer "F.Cu") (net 14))
 (segment (start 143.62 64.4) (end 143.58 64.44) (width 0.2) (layer "F.Cu") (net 14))
 (via (at 143.62 64.4) (size 0.6) (drill 0.3) (layers "F.Cu" "B.Cu") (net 14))
 (via (at 135.17 64.26) (size 0.6) (drill 0.3) (layers "F.Cu" "B.Cu") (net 14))
 (segment (start 135.17 64.26) (end 143.48 64.26) (width 0.2) (layer "B.Cu") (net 14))
 (segment (start 143.48 64.26) (end 143.62 64.4) (width 0.2) (layer "B.Cu") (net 14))
 (segment (start 122.315 59.34) (end 139.54 59.34) (width 0.2) (layer "F.Cu") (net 3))
 (segment (start 153.74 58.9) (end 153.74 53.77) (width 0.2) (layer "F.Cu") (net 3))
 (segment (start 153.56 59.08) (end 153.74 58.9) (width 0.2) (layer "F.Cu") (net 3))
 (segment (start 139.54 59.34) (end 139.56 59.36) (width 0.2) (layer "F.Cu") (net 3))
 (segment (start 153.56 59.36) (end 153.56 59.08) (width 0.2) (layer "F.Cu") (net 3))
 (via (at 153.56 59.36) (size 0.6) (drill 0.3) (layers "F.Cu" "B.Cu") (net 3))
 (via (at 139.56 59.36) (size 0.6) (drill 0.3) (layers "F.Cu" "B.Cu") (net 3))
 (segment (start 139.56 59.36) (end 153.56 59.36) (width 0.2) (layer "B.Cu") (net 3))
 (segment (start 103.245 78.39) (end 120.333686 78.39) (width 0.2) (layer "F.Cu") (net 4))
 (segment (start 151.32 66.74) (end 151.2 66.62) (width 0.2) (layer "F.Cu") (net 4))
 (segment (start 131.983686 66.74) (end 132 66.74) (width 0.2) (layer "F.Cu") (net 4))
 (segment (start 120.333686 78.39) (end 131.983686 66.74) (width 0.2) (layer "F.Cu") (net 4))
 (segment (start 151.2 66.62) (end 151.2 53.77) (width 0.2) (layer "F.Cu") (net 4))
 (via (at 132 66.74) (size 0.6) (drill 0.3) (layers "F.Cu" "B.Cu") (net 4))
 (via (at 151.32 66.74) (size 0.6) (drill 0.3) (layers "F.Cu" "B.Cu") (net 4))
 (segment (start 132 66.74) (end 151.32 66.74) (width 0.2) (layer "B.Cu") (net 4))
 (segment (start 145.531 56.899) (end 148.66 53.77) (width 0.2) (layer "F.Cu") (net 2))
 (segment (start 122.315 78.39) (end 143.806 56.899) (width 0.2) (layer "F.Cu") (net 2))
 (segment (start 143.806 56.899) (end 145.531 56.899) (width 0.2) (layer "F.Cu") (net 2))
 (segment (start 141.365 76.965) (end 141.52 76.81) (width 0.2) (layer "F.Cu") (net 5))
 (segment (start 141.365 78.39) (end 141.365 76.965) (width 0.2) (layer "F.Cu") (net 5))
 (segment (start 142.22 60.95) (end 145.67 57.5) (width 0.2) (layer "F.Cu") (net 5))
 (segment (start 142.22 67.81) (end 142.22 60.95) (width 0.2) (layer "F.Cu") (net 5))
 (segment (start 146.18 53.83) (end 146.12 53.77) (width 0.2) (layer "F.Cu") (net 5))
 (segment (start 146.18 55.31) (end 146.18 53.83) (width 0.2) (layer "F.Cu") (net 5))
 (via (at 141.52 76.81) (size 0.6) (drill 0.3) (layers "F.Cu" "B.Cu") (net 5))
 (via (at 146.18 55.31) (size 0.6) (drill 0.3) (layers "F.Cu" "B.Cu") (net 5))
 (via (at 142.22 67.81) (size 0.6) (drill 0.3) (layers "F.Cu" "B.Cu") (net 5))
 (via (at 145.67 57.5) (size 0.6) (drill 0.3) (layers "F.Cu" "B.Cu") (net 5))
 (segment (start 145.67 57.5) (end 145.67 55.82) (width 0.2) (layer "B.Cu") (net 5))
 (segment (start 141.52 76.81) (end 142.22 76.11) (width 0.2) (layer "B.Cu") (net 5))
 (segment (start 145.67 55.82) (end 146.18 55.31) (width 0.2) (layer "B.Cu") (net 5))
 (segment (start 142.22 76.11) (end 142.22 67.81) (width 0.2) (layer "B.Cu") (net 5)))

